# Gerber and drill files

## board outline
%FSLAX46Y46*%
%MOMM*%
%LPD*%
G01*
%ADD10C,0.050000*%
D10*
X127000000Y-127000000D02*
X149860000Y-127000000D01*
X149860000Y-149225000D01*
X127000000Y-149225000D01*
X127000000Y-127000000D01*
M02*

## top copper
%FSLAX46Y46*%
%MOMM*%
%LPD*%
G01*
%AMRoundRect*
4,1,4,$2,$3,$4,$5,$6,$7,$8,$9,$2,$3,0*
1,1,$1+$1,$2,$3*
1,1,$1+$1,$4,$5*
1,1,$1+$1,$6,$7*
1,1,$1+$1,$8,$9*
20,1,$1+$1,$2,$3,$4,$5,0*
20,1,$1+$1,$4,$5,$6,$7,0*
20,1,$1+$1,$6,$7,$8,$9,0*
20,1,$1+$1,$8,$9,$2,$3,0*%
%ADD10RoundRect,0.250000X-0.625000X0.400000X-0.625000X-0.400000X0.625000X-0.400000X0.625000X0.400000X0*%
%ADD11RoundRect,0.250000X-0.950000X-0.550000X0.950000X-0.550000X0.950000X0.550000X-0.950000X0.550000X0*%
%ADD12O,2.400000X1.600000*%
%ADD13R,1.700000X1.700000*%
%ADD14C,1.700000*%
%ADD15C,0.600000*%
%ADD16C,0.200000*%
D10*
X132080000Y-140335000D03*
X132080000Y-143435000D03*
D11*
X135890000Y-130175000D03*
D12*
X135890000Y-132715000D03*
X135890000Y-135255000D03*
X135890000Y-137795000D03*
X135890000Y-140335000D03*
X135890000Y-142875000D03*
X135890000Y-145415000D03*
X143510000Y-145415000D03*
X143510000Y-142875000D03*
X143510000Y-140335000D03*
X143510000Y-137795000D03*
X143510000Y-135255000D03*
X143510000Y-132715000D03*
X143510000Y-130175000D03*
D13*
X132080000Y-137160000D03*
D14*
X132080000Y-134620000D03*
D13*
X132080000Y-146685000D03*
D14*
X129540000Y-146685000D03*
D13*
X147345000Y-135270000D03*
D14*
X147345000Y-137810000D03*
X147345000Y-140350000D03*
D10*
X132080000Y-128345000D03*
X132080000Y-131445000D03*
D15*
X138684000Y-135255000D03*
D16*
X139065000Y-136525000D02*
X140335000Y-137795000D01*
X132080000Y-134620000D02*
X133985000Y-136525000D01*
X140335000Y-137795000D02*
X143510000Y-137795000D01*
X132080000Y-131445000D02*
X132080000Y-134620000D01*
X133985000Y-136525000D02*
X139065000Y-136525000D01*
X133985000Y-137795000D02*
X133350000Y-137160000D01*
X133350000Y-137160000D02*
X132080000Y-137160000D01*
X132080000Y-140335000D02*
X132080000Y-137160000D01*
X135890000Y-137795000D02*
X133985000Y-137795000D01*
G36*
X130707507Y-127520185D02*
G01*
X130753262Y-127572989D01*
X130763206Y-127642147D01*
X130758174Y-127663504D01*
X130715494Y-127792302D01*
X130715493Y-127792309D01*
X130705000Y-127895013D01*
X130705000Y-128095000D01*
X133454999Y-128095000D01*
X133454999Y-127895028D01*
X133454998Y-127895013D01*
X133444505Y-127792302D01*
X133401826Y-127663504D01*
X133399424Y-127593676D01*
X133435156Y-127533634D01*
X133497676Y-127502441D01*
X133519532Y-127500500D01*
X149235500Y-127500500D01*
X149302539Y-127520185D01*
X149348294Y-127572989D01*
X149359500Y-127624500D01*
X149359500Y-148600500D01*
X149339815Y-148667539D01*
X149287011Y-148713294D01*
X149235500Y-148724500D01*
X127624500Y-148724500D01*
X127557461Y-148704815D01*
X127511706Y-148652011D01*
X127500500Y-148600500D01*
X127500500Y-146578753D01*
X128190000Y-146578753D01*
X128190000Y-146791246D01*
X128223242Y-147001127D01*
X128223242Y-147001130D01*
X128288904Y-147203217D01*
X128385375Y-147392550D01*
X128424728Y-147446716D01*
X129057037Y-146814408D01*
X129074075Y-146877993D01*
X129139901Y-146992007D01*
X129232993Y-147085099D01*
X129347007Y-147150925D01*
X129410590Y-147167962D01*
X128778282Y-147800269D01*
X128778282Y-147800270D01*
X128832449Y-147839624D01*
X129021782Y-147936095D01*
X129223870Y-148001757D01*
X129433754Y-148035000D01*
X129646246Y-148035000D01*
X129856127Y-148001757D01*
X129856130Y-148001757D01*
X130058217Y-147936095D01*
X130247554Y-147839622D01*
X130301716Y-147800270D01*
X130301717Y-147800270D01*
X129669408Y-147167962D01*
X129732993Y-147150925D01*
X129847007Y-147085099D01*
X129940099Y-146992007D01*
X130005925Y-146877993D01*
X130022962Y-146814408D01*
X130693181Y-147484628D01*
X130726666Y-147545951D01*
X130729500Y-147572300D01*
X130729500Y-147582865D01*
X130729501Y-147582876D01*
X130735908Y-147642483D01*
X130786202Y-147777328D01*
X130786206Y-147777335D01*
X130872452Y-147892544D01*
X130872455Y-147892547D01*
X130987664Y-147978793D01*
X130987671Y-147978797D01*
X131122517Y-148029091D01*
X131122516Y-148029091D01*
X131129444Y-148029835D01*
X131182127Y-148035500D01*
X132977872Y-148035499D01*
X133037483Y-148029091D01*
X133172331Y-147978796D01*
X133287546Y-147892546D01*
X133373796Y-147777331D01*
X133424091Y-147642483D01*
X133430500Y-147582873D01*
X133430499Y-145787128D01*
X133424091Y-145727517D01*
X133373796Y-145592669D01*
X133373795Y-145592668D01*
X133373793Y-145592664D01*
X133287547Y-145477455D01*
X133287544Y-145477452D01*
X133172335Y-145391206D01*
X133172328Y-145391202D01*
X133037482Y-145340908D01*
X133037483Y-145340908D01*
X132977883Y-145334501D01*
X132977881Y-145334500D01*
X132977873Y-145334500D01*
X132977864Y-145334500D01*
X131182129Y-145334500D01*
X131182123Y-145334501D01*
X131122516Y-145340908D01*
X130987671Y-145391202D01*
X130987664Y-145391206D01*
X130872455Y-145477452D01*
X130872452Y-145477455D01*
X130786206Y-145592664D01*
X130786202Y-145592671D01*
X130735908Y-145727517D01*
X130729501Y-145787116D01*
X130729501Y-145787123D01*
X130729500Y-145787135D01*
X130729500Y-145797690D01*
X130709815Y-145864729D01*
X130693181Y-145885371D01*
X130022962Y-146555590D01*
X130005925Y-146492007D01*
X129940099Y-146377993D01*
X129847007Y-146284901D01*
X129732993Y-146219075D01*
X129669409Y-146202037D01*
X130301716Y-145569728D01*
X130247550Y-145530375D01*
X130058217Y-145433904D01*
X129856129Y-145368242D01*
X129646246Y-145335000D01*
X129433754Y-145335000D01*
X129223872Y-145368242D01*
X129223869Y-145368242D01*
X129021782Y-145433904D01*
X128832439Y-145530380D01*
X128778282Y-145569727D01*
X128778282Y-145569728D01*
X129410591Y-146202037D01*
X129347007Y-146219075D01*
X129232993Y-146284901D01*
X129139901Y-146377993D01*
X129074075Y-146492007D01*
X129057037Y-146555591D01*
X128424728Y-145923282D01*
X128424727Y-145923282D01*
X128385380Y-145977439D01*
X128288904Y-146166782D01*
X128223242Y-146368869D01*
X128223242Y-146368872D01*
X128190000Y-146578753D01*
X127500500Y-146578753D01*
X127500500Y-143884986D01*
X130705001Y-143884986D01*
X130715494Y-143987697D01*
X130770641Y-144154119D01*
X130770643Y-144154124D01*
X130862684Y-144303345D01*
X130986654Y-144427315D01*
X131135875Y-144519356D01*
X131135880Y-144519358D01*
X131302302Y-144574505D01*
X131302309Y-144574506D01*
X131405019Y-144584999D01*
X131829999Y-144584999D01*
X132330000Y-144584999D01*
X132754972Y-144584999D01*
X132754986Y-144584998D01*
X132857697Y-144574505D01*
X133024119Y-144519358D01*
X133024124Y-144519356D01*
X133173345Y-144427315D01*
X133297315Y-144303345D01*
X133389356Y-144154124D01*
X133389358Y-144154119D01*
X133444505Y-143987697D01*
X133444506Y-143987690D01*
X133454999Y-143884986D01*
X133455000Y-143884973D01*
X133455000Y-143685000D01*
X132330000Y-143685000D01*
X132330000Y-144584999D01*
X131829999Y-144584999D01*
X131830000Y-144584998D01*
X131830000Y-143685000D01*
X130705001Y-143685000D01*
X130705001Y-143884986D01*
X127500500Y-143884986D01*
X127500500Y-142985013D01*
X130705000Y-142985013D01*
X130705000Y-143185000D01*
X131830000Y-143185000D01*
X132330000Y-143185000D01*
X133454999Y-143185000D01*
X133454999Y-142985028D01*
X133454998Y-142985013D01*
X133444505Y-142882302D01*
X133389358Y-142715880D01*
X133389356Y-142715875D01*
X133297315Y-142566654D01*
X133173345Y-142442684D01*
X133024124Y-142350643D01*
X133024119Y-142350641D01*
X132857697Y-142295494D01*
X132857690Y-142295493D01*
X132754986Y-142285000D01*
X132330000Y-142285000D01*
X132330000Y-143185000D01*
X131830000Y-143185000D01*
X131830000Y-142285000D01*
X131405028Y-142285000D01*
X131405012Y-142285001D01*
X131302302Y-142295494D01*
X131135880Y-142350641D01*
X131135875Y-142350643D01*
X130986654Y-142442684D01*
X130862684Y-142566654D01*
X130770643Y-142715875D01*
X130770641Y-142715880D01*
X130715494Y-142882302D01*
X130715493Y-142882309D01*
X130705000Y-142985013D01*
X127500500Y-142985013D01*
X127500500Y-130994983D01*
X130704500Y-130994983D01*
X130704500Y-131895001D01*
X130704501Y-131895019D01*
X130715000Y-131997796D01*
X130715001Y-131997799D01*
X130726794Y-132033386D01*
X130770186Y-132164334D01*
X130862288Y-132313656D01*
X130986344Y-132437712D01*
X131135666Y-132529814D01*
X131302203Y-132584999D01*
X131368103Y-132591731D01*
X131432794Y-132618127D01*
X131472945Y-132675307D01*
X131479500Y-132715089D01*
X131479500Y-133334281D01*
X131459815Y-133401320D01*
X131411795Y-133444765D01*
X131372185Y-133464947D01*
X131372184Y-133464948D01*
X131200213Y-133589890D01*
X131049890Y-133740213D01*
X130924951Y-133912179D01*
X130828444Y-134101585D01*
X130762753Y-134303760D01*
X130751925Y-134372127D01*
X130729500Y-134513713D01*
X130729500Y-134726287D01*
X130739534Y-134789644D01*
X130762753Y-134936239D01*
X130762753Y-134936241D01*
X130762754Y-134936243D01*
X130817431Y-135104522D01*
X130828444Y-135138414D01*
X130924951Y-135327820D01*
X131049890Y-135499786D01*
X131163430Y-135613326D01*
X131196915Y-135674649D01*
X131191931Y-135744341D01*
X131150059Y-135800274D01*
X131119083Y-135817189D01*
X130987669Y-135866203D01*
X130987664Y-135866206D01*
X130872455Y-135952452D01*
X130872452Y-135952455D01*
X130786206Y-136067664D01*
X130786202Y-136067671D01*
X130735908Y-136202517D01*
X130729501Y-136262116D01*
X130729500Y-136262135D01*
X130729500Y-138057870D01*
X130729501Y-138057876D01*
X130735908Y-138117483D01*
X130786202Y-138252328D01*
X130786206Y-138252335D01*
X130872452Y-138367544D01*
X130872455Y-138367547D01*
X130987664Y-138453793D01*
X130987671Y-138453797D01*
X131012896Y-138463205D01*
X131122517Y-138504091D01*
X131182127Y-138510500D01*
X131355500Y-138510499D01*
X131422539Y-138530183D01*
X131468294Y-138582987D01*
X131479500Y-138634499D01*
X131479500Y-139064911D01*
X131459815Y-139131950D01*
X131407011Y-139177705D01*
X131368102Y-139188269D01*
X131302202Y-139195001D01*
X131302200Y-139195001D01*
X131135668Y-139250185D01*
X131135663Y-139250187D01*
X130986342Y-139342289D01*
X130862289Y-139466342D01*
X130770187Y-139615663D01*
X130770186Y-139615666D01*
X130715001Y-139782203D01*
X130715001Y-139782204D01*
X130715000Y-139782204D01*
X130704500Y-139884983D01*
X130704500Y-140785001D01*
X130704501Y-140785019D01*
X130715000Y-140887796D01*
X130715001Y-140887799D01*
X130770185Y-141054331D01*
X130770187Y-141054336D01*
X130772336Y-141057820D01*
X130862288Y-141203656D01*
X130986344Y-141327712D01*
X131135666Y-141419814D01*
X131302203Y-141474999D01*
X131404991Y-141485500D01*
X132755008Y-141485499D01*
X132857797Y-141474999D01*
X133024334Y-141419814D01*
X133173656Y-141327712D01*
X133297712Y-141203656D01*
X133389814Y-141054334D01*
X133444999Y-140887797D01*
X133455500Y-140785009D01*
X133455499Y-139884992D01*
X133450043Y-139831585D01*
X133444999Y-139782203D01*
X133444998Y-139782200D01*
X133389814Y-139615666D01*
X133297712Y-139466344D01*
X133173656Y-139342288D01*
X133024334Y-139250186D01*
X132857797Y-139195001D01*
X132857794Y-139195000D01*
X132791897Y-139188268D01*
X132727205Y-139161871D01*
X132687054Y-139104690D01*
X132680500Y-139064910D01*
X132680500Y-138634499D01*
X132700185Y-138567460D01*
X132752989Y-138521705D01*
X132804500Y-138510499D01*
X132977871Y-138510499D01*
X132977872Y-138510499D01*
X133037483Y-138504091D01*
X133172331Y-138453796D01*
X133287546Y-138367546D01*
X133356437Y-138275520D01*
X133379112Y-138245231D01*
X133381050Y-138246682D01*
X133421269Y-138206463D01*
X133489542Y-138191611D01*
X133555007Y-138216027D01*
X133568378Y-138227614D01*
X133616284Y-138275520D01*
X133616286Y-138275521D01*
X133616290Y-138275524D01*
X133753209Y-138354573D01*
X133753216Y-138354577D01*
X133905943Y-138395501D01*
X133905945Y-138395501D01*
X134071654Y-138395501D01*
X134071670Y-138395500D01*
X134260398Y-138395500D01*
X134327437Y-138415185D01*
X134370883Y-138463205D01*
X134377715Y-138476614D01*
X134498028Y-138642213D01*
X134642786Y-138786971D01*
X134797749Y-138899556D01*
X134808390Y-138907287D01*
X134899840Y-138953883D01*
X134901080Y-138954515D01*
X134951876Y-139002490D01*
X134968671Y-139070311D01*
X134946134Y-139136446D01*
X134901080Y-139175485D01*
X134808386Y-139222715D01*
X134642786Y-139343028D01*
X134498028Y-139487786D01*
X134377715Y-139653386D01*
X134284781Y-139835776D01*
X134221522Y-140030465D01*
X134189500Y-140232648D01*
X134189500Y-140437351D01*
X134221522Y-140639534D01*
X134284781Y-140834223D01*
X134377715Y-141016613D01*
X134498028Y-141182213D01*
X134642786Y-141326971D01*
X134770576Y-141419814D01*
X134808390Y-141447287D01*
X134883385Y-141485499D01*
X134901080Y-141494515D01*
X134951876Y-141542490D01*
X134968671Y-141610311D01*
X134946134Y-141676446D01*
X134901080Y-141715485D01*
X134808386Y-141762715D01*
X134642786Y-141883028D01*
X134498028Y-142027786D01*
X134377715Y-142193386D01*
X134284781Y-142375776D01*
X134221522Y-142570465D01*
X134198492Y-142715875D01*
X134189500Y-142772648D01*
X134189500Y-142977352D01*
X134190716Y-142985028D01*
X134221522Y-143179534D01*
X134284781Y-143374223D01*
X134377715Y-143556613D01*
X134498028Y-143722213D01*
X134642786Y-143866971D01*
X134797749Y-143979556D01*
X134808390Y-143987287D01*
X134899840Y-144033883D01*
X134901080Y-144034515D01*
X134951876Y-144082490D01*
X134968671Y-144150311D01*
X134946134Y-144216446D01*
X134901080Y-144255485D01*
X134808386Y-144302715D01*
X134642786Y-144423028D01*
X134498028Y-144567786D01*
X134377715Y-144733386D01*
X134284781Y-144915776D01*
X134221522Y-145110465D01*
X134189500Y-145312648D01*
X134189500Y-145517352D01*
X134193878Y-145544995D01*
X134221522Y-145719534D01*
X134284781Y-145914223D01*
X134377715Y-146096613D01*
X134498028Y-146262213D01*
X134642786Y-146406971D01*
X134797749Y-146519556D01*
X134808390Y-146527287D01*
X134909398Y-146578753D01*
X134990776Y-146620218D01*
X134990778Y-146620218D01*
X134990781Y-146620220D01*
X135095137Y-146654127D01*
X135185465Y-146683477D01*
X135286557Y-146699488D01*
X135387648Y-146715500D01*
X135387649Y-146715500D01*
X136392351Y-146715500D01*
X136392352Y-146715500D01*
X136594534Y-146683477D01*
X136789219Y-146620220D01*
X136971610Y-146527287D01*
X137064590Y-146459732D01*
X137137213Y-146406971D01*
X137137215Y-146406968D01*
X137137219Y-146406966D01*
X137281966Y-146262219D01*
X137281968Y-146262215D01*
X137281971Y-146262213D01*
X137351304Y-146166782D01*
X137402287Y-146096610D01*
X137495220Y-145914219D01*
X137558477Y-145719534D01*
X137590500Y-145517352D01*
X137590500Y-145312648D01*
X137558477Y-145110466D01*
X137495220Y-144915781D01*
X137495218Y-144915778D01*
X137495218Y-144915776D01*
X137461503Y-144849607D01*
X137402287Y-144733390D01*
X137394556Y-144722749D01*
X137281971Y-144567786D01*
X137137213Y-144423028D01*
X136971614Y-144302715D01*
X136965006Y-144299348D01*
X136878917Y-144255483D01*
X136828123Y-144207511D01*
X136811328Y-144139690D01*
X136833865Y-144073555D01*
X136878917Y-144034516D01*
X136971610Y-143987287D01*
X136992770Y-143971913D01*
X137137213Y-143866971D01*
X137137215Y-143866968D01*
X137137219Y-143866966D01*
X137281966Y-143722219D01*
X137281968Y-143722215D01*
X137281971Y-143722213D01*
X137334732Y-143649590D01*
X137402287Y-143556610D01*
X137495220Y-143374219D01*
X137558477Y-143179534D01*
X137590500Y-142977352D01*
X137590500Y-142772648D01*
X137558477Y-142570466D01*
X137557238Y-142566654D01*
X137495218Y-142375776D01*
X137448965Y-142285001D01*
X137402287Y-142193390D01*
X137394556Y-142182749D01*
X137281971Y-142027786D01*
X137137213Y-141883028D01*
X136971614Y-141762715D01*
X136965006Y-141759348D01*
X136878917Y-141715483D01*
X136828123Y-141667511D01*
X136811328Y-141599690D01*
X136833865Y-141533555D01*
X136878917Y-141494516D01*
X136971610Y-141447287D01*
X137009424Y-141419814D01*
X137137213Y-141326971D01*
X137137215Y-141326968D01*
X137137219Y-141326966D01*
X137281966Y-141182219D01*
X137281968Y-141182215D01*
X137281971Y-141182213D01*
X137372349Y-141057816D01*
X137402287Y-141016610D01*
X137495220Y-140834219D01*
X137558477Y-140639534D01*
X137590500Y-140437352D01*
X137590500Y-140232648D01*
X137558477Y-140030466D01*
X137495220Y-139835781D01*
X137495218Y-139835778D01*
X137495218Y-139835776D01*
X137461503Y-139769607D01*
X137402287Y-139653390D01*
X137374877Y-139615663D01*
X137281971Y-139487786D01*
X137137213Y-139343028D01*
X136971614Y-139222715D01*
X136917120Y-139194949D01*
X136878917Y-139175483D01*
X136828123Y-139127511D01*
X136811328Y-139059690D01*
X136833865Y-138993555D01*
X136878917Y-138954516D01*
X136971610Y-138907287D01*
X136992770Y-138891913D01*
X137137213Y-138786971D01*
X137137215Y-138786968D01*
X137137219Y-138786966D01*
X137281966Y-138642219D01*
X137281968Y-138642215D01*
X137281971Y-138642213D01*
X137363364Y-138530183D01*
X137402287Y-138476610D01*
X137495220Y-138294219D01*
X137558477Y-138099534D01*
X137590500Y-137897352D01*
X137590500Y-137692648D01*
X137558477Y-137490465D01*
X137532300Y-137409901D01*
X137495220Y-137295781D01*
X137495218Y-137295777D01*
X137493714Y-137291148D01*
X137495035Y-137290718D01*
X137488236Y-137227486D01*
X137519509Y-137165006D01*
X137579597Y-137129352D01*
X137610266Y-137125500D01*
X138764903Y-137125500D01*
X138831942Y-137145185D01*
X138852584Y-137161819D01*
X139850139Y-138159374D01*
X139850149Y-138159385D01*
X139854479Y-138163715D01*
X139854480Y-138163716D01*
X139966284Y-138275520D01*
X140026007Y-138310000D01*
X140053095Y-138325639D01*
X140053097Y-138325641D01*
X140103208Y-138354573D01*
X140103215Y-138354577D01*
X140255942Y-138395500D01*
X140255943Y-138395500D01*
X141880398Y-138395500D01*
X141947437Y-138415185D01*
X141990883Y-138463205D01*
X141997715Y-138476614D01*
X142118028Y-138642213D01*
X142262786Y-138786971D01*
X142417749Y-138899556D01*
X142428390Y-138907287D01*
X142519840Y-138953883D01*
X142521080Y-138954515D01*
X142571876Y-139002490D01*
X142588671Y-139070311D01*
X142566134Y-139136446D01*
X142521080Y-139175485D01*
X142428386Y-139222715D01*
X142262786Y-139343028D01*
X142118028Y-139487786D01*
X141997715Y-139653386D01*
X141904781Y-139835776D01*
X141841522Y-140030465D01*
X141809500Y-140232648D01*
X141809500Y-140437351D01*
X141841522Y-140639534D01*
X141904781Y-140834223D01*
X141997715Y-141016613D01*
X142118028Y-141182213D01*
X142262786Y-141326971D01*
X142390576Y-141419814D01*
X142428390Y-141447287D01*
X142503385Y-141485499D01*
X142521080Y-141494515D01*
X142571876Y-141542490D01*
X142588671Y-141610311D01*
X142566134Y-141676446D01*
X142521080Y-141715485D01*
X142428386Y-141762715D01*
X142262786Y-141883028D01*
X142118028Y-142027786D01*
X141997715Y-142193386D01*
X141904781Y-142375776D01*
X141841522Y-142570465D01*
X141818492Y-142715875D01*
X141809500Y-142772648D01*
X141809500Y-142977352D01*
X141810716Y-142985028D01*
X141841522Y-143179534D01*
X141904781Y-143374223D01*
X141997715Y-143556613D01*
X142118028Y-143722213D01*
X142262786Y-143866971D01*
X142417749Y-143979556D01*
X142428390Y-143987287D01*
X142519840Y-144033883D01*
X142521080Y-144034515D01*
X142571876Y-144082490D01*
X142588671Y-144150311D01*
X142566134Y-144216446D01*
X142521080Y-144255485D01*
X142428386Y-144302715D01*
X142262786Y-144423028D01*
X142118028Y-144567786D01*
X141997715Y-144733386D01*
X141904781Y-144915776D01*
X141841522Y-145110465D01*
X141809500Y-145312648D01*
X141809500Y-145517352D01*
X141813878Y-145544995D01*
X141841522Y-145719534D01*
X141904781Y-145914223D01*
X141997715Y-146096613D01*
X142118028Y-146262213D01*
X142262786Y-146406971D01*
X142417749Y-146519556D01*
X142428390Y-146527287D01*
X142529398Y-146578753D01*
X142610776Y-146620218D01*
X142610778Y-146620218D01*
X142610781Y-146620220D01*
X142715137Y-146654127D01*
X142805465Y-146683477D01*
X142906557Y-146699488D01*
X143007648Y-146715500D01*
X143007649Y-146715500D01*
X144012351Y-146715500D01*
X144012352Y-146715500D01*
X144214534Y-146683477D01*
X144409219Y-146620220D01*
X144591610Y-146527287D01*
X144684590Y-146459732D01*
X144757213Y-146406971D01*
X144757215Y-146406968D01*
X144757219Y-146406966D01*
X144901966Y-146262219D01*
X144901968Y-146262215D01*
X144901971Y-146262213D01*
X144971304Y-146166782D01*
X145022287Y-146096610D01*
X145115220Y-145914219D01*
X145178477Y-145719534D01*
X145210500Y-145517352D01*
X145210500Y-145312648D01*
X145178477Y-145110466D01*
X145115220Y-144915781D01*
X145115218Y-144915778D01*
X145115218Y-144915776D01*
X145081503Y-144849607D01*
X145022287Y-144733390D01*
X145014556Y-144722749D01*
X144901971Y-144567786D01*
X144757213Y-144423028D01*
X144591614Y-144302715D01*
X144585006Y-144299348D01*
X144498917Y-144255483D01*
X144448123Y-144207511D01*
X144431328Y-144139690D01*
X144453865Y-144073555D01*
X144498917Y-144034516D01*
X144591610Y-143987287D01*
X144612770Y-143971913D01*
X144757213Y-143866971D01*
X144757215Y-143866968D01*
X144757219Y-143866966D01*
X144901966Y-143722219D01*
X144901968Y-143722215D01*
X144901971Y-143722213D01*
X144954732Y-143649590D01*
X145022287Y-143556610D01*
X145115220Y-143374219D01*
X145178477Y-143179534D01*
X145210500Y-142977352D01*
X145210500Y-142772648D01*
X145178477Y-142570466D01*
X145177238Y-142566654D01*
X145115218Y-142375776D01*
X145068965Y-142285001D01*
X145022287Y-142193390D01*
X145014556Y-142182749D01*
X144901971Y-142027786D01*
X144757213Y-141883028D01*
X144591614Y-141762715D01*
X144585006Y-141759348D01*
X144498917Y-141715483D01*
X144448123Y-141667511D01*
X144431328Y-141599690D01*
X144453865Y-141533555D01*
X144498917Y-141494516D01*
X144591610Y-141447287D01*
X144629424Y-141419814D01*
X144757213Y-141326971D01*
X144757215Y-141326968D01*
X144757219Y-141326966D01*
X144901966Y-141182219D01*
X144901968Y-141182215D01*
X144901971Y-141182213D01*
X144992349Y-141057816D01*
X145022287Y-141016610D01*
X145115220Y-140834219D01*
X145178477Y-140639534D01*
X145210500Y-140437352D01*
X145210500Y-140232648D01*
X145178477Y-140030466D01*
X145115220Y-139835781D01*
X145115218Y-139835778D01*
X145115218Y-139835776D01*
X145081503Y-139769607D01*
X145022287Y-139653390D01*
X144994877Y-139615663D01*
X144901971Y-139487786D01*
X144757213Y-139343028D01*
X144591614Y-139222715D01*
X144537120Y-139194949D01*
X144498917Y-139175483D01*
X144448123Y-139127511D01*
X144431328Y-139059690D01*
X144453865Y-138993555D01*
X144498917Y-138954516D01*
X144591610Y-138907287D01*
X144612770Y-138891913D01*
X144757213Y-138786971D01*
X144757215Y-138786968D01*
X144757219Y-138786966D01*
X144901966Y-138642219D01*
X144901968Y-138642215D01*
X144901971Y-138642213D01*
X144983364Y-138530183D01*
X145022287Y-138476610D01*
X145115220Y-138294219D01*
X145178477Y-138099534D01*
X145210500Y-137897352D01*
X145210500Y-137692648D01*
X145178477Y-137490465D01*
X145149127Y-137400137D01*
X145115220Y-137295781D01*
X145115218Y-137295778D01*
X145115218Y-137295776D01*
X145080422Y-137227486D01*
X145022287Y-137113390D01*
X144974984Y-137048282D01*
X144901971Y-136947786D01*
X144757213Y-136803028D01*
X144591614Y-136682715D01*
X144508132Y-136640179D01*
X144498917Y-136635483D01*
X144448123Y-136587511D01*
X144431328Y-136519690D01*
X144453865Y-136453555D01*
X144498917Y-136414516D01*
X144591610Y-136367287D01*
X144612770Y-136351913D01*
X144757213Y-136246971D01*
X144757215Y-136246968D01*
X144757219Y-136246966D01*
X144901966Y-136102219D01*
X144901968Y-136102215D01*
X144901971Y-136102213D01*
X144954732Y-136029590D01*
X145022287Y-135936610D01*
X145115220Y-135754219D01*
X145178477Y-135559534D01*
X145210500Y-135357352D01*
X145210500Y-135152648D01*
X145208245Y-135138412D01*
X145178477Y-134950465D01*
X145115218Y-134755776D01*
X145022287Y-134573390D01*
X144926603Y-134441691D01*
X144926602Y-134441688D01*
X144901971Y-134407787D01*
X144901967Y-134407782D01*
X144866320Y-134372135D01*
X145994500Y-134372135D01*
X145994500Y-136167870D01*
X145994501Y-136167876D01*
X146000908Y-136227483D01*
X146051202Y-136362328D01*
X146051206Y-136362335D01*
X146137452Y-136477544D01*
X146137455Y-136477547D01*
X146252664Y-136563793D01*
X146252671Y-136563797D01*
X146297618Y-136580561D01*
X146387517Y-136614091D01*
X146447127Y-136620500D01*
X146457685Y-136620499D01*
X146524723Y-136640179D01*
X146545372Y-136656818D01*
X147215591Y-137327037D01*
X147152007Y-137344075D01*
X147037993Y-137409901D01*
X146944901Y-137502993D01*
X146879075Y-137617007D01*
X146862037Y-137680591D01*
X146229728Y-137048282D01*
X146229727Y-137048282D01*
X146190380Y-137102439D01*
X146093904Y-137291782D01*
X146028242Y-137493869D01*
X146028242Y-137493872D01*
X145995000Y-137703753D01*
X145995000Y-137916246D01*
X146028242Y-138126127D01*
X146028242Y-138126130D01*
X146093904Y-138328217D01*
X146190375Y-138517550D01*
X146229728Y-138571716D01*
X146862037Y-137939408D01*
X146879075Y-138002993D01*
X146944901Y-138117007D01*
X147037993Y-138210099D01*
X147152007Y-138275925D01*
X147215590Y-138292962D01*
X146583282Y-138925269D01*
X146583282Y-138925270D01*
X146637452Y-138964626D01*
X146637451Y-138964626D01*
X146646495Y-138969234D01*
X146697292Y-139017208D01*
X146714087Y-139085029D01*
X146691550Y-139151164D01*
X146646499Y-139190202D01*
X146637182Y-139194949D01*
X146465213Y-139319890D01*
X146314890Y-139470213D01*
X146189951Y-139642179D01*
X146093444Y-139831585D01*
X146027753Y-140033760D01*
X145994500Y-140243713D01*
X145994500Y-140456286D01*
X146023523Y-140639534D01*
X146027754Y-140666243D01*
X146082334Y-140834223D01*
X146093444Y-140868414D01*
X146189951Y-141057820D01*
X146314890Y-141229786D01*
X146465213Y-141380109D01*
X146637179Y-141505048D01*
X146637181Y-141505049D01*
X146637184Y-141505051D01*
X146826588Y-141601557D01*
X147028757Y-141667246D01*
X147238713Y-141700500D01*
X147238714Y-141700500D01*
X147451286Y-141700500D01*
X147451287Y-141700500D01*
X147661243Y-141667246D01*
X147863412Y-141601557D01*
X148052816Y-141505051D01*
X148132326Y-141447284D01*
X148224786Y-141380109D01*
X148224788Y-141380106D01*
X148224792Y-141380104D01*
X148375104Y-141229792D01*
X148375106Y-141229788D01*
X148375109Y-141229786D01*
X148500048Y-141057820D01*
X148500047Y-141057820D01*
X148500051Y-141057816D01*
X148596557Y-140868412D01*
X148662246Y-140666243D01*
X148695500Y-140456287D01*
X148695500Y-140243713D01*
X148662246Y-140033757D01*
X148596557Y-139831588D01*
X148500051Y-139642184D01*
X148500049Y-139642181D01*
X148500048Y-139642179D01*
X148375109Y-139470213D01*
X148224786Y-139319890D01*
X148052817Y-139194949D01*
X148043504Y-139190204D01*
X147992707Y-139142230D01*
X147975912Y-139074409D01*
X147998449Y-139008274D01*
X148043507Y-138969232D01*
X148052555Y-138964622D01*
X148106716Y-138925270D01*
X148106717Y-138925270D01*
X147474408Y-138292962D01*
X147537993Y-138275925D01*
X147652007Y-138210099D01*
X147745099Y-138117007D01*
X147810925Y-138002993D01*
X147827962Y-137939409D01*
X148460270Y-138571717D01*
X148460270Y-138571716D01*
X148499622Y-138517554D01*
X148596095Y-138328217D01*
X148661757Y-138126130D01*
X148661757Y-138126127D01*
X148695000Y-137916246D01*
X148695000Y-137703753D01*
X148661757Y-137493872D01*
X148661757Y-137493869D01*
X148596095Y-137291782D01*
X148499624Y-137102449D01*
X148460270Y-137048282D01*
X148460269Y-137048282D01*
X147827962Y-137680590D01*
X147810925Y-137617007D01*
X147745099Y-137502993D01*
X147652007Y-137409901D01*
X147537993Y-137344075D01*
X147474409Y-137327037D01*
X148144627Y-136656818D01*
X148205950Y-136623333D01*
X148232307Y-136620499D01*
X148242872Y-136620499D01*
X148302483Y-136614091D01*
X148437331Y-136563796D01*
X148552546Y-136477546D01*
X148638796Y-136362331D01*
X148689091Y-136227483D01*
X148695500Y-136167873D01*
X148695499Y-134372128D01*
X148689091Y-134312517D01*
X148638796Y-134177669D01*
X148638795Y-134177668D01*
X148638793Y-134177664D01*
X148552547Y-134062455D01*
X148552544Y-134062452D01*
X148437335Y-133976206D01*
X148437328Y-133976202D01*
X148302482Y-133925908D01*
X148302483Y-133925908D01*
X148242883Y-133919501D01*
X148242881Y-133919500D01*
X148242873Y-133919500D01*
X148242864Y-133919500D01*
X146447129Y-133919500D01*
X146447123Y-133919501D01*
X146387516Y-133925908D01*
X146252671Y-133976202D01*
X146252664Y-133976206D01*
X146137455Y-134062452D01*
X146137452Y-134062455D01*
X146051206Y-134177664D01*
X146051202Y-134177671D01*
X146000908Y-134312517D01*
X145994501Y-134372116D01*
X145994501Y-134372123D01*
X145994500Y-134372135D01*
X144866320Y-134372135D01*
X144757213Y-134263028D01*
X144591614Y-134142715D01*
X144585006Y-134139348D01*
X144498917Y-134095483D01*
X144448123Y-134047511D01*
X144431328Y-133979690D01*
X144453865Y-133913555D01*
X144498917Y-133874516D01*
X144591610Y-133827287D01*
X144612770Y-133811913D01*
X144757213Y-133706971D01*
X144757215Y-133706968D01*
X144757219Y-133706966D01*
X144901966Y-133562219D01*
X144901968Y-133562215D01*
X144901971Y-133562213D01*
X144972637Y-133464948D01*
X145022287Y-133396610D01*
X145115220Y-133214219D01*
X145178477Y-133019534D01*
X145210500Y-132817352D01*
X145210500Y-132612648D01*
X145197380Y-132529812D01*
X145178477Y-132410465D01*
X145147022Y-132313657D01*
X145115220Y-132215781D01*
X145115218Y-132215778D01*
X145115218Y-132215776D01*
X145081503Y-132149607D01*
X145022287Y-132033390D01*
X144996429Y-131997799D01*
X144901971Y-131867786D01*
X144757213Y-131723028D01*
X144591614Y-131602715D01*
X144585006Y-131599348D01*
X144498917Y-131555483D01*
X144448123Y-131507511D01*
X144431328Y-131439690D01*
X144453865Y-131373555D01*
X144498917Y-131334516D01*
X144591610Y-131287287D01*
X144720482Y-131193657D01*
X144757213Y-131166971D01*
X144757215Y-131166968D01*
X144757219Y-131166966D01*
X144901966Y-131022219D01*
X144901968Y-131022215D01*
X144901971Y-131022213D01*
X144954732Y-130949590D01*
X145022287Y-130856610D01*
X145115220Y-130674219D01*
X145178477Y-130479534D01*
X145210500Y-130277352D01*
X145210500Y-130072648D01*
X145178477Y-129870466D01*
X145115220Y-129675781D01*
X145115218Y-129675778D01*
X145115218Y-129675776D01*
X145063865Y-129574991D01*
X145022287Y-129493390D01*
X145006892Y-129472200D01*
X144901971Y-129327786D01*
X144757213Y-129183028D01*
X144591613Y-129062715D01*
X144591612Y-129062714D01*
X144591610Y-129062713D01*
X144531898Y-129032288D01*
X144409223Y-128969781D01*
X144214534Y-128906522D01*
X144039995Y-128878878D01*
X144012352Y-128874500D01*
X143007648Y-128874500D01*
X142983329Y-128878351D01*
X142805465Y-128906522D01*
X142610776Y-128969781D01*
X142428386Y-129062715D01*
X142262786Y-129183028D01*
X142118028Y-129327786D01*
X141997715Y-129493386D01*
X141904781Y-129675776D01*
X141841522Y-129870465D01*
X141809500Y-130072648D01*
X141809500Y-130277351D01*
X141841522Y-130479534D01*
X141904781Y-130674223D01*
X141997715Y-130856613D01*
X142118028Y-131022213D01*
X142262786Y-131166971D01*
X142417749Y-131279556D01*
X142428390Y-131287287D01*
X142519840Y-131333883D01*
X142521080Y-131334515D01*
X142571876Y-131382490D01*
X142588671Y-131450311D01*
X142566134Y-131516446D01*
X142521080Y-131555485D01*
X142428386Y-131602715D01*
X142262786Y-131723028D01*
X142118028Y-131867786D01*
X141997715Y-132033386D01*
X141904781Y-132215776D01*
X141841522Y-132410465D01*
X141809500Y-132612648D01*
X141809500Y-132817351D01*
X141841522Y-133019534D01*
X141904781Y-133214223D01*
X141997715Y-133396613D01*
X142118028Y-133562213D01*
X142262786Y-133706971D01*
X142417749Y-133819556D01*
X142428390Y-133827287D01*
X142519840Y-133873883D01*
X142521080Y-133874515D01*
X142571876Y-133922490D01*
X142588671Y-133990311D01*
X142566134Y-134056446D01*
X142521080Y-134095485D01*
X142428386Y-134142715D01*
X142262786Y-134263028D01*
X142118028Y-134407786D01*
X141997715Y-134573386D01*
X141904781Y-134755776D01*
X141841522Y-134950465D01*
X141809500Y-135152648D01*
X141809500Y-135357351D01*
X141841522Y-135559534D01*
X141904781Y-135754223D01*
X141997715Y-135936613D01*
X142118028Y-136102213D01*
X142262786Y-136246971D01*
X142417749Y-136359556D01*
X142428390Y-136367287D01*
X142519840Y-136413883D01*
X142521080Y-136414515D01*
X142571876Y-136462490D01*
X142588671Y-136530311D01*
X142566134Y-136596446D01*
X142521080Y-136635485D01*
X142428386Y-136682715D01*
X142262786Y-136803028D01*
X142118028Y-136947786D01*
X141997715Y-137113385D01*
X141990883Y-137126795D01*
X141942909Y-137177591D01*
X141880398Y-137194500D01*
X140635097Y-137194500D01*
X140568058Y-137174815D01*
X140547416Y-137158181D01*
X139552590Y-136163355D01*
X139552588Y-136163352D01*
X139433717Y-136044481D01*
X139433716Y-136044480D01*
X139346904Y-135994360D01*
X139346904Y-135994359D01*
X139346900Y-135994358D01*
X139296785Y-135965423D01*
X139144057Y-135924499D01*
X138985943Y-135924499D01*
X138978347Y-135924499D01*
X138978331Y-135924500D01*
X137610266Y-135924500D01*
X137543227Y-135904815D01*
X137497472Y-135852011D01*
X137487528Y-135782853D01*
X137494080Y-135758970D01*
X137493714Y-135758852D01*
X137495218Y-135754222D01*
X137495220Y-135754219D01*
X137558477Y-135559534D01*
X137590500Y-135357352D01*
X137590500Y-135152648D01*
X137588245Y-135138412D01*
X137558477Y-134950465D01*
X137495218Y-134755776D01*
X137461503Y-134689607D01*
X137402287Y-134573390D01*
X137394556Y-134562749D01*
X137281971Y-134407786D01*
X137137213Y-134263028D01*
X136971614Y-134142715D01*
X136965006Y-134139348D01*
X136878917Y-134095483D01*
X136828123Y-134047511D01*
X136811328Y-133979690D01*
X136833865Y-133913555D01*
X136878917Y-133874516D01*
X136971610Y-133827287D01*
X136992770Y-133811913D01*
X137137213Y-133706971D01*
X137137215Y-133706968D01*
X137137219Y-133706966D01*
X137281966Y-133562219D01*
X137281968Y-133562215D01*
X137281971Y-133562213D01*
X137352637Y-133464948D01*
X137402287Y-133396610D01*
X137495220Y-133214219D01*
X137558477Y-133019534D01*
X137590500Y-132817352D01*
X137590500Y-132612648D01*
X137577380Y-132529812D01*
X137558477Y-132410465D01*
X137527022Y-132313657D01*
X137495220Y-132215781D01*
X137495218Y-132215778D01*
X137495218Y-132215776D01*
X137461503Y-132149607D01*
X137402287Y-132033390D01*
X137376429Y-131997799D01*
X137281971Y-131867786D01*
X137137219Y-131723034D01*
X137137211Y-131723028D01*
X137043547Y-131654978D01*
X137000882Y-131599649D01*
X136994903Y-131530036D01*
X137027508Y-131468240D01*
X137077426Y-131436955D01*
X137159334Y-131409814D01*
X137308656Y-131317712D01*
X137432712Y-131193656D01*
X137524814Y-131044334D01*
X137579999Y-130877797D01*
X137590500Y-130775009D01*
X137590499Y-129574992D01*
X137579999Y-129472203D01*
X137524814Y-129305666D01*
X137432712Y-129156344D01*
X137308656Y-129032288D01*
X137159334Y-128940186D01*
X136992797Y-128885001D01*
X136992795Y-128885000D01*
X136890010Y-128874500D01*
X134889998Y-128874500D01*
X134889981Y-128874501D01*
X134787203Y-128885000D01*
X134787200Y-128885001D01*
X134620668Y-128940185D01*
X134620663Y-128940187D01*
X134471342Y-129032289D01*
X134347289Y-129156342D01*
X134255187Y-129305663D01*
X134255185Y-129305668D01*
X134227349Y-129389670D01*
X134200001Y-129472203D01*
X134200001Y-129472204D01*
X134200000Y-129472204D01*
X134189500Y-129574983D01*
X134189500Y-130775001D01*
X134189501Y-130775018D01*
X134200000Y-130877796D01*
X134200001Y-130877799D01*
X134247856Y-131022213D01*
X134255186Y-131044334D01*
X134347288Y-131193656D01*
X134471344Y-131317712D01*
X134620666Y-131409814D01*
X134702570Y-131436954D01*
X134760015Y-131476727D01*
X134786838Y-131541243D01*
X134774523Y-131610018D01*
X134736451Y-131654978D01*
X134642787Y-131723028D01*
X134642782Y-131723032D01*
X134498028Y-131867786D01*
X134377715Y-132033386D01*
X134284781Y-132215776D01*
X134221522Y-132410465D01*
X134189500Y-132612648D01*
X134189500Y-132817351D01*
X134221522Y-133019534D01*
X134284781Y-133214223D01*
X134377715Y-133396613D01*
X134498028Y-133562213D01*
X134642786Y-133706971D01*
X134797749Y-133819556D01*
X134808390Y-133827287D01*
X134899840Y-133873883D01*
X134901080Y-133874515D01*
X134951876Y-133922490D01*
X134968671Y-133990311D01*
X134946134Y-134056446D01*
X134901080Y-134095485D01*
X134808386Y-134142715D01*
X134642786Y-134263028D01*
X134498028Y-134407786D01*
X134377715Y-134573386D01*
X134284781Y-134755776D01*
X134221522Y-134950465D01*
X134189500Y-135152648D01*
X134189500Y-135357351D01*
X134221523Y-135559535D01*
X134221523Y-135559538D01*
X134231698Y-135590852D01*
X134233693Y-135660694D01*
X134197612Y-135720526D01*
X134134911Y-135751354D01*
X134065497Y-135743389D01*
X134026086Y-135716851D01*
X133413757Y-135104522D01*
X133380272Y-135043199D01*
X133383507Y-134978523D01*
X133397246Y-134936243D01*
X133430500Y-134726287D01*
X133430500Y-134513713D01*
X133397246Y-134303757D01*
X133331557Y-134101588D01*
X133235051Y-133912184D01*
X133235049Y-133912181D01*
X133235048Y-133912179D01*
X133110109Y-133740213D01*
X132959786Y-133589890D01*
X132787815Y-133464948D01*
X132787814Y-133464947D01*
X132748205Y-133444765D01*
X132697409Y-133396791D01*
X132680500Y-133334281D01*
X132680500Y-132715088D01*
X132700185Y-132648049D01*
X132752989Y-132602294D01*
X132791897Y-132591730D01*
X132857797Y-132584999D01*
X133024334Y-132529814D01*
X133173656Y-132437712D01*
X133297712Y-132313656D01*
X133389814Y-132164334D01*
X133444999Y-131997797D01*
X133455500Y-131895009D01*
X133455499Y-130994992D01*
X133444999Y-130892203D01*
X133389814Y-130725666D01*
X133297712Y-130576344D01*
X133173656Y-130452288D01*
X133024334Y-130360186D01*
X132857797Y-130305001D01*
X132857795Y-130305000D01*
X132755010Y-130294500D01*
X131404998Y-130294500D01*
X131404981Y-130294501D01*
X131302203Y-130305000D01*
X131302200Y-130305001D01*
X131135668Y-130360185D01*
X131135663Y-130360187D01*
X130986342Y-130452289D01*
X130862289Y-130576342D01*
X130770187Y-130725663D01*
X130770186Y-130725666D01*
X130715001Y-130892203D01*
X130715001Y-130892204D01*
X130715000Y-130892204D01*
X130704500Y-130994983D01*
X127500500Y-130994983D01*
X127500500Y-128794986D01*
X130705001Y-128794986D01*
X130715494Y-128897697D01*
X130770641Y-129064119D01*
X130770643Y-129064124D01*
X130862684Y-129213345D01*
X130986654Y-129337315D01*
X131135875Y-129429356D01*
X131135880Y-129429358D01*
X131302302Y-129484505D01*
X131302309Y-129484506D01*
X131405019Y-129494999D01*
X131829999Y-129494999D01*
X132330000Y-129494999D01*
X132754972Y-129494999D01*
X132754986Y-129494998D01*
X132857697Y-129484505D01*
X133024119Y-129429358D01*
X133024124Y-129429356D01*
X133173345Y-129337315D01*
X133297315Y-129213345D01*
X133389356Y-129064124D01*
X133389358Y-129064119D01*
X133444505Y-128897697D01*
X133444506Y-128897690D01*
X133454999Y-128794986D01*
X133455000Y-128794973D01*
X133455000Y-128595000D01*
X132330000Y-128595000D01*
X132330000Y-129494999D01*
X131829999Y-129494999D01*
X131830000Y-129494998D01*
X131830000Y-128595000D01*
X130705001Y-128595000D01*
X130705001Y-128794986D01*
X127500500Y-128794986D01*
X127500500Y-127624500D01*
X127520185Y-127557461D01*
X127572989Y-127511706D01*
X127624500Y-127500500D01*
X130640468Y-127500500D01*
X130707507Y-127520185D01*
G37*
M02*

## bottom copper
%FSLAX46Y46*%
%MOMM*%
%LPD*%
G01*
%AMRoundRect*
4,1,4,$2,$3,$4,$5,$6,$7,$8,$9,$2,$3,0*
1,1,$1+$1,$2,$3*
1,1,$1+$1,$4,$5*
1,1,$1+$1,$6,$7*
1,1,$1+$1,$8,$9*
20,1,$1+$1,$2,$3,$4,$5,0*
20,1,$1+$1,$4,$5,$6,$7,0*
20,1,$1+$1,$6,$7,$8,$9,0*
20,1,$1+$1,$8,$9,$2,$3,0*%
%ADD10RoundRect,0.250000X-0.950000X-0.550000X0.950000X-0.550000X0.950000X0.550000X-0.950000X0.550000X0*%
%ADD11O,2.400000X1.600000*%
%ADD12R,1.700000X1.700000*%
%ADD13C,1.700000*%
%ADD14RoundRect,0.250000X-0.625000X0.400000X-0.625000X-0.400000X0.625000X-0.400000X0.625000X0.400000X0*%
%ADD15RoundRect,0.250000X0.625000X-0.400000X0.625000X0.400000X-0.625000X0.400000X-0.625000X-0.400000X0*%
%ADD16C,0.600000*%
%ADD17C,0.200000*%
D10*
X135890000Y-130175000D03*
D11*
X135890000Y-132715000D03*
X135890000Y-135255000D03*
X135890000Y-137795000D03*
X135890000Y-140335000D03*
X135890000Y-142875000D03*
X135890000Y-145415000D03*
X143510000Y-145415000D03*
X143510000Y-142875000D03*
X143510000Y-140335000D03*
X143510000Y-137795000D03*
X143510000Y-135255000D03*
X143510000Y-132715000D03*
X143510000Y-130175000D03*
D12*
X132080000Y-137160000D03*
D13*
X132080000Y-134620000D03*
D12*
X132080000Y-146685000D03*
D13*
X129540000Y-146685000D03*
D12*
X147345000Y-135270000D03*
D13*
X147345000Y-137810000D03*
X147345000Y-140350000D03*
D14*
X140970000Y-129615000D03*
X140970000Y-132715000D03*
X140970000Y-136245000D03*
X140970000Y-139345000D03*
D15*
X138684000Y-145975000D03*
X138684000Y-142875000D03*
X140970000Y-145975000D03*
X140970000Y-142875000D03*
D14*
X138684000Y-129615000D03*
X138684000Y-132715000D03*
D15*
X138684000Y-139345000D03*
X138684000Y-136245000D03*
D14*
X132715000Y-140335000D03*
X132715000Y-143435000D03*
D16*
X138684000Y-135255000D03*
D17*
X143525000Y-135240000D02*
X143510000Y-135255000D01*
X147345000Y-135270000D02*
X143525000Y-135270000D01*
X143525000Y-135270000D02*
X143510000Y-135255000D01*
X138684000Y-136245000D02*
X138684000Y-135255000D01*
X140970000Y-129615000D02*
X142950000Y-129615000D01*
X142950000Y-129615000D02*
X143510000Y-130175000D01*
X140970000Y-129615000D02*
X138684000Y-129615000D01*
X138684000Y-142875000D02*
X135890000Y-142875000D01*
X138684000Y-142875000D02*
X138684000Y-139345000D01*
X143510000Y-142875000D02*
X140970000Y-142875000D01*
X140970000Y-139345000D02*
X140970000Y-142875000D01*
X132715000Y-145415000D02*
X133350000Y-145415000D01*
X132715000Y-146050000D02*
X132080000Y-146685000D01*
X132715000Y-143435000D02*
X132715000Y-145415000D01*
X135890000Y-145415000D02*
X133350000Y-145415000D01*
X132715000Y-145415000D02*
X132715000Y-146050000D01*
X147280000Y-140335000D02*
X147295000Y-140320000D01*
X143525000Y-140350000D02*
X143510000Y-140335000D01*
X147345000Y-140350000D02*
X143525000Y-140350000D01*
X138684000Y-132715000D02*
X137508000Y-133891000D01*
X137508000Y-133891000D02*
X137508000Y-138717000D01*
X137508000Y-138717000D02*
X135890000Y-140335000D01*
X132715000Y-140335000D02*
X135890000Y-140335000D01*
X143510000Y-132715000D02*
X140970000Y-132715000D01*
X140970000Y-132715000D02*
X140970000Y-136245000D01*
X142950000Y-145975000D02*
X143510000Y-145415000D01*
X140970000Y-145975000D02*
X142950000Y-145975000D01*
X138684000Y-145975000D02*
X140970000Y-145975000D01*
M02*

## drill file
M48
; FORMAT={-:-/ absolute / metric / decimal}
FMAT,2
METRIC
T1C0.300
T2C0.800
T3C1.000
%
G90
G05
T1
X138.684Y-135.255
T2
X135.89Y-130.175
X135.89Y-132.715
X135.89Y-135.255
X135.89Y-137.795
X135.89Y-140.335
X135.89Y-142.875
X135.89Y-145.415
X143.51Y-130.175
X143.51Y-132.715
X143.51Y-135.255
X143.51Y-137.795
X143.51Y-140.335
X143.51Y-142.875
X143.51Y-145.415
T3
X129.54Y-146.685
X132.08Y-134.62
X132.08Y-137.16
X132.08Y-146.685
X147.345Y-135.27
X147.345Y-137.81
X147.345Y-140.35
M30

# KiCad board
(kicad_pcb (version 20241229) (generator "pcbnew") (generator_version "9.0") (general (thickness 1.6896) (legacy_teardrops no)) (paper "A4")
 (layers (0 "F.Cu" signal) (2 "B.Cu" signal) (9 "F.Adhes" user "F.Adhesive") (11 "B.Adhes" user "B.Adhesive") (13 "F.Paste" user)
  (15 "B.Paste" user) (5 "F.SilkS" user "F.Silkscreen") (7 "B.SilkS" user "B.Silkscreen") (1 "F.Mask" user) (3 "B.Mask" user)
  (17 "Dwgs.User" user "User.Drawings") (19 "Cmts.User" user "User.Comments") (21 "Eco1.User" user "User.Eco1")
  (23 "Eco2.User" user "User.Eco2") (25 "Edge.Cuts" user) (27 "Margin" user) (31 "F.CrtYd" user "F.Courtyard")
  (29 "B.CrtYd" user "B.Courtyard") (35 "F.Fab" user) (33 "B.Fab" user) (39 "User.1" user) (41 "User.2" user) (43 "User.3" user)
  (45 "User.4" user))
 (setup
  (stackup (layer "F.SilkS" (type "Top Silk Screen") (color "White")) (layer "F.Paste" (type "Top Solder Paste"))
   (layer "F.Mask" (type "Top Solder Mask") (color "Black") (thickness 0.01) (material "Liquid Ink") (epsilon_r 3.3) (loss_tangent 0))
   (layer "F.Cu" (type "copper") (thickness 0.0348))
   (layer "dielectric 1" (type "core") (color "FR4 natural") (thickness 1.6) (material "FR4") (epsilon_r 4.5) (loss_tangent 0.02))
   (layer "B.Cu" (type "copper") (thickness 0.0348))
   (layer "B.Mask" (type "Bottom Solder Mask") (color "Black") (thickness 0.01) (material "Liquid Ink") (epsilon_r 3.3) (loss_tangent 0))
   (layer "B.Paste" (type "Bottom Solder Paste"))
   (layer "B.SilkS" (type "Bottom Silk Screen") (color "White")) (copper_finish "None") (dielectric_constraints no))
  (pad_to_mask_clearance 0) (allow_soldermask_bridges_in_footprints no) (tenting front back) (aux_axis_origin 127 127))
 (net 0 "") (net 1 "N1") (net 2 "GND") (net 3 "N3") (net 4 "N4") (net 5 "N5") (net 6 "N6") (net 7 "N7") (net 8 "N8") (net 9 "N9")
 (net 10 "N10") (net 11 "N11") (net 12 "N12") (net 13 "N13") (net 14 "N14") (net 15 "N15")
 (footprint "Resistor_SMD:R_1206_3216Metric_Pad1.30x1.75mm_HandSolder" (layer "F.Cu") (at 132.08 141.885 -90)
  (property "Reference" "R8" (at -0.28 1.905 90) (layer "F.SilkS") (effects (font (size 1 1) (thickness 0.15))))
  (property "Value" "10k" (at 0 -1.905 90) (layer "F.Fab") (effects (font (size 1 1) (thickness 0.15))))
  (pad "1" smd roundrect (at -1.55 0 270) (size 1.3 1.75) (layers "F.Cu" "F.Mask" "F.Paste") (roundrect_rratio 0.192308) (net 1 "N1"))
  (pad "2" smd roundrect (at 1.55 0 270) (size 1.3 1.75) (layers "F.Cu" "F.Mask" "F.Paste") (roundrect_rratio 0.192308) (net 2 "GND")))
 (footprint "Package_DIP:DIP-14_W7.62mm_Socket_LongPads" (layer "F.Cu") (at 135.89 130.175)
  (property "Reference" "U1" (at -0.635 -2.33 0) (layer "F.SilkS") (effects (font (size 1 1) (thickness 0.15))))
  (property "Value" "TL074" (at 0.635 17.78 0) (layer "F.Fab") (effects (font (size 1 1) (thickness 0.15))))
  (pad "1" thru_hole roundrect (at 0 0) (size 2.4 1.6) (drill 0.8) (layers "*.Cu" "*.Mask") (remove_unused_layers no)
   (roundrect_rratio 0.15625) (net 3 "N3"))
  (pad "2" thru_hole oval (at 0 2.54) (size 2.4 1.6) (drill 0.8) (layers "*.Cu" "*.Mask") (remove_unused_layers no) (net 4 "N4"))
  (pad "3" thru_hole oval (at 0 5.08) (size 2.4 1.6) (drill 0.8) (layers "*.Cu" "*.Mask") (remove_unused_layers no) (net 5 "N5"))
  (pad "4" thru_hole oval (at 0 7.62) (size 2.4 1.6) (drill 0.8) (layers "*.Cu" "*.Mask") (remove_unused_layers no) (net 1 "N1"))
  (pad "5" thru_hole oval (at 0 10.16) (size 2.4 1.6) (drill 0.8) (layers "*.Cu" "*.Mask") (remove_unused_layers no) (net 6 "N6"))
  (pad "6" thru_hole oval (at 0 12.7) (size 2.4 1.6) (drill 0.8) (layers "*.Cu" "*.Mask") (remove_unused_layers no) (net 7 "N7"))
  (pad "7" thru_hole oval (at 0 15.24) (size 2.4 1.6) (drill 0.8) (layers "*.Cu" "*.Mask") (remove_unused_layers no) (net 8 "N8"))
  (pad "8" thru_hole oval (at 7.62 15.24) (size 2.4 1.6) (drill 0.8) (layers "*.Cu" "*.Mask") (remove_unused_layers no) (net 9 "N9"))
  (pad "9" thru_hole oval (at 7.62 12.7) (size 2.4 1.6) (drill 0.8) (layers "*.Cu" "*.Mask") (remove_unused_layers no) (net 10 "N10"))
  (pad "10" thru_hole oval (at 7.62 10.16) (size 2.4 1.6) (drill 0.8) (layers "*.Cu" "*.Mask") (remove_unused_layers no) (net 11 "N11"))
  (pad "11" thru_hole oval (at 7.62 7.62) (size 2.4 1.6) (drill 0.8) (layers "*.Cu" "*.Mask") (remove_unused_layers no) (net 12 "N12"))
  (pad "12" thru_hole oval (at 7.62 5.08) (size 2.4 1.6) (drill 0.8) (layers "*.Cu" "*.Mask") (remove_unused_layers no) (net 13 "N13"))
  (pad "13" thru_hole oval (at 7.62 2.54) (size 2.4 1.6) (drill 0.8) (layers "*.Cu" "*.Mask") (remove_unused_layers no) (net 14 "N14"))
  (pad "14" thru_hole oval (at 7.62 0) (size 2.4 1.6) (drill 0.8) (layers "*.Cu" "*.Mask") (remove_unused_layers no) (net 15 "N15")))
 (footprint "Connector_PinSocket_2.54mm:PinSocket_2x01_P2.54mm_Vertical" (layer "F.Cu") (at 132.08 137.16 -90)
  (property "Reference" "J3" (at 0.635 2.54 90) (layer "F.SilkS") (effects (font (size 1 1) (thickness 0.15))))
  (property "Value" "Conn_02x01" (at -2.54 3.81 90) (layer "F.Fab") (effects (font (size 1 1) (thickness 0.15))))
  (pad "1" thru_hole rect (at 0 0 270) (size 1.7 1.7) (drill 1) (layers "*.Cu" "*.Mask") (remove_unused_layers no) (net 1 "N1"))
  (pad "2" thru_hole circle (at -2.54 0 270) (size 1.7 1.7) (drill 1) (layers "*.Cu" "*.Mask") (remove_unused_layers no) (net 12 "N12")))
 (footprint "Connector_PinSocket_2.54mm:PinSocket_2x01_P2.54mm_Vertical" (layer "F.Cu") (at 132.08 146.685)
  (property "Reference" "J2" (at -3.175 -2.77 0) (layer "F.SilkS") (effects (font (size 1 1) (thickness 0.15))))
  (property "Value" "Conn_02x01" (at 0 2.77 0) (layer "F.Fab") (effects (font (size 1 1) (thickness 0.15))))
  (pad "1" thru_hole rect (at 0 0) (size 1.7 1.7) (drill 1) (layers "*.Cu" "*.Mask") (remove_unused_layers no) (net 8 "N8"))
  (pad "2" thru_hole circle (at -2.54 0) (size 1.7 1.7) (drill 1) (layers "*.Cu" "*.Mask") (remove_unused_layers no) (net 2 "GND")))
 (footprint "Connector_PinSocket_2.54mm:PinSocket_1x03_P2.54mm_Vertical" (layer "F.Cu") (at 147.345 135.27)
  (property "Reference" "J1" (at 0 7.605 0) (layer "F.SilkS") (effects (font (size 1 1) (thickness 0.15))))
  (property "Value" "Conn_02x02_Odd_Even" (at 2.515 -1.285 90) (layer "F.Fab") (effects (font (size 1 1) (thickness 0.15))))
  (pad "1" thru_hole rect (at 0 0) (size 1.7 1.7) (drill 1) (layers "*.Cu" "*.Mask") (remove_unused_layers no) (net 13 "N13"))
  (pad "2" thru_hole circle (at 0 2.54) (size 1.7 1.7) (drill 1) (layers "*.Cu" "*.Mask") (remove_unused_layers no) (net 2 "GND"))
  (pad "3" thru_hole circle (at 0 5.08) (size 1.7 1.7) (drill 1) (layers "*.Cu" "*.Mask") (remove_unused_layers no) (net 11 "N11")))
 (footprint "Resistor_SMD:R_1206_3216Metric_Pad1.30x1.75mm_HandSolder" (layer "F.Cu") (at 132.08 129.895 -90)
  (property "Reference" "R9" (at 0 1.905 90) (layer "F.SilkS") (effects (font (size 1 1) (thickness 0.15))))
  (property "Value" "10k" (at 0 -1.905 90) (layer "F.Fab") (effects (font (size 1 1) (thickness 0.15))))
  (pad "1" smd roundrect (at -1.55 0 270) (size 1.3 1.75) (layers "F.Cu" "F.Mask" "F.Paste") (roundrect_rratio 0.192308) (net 2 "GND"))
  (pad "2" smd roundrect (at 1.55 0 270) (size 1.3 1.75) (layers "F.Cu" "F.Mask" "F.Paste") (roundrect_rratio 0.192308) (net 12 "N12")))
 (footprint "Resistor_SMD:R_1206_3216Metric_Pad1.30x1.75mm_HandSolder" (layer "B.Cu") (at 140.97 131.165 -90)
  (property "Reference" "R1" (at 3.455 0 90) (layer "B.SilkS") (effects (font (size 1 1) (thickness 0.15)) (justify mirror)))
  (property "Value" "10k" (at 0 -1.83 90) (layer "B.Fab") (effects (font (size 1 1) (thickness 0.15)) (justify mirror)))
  (pad "1" smd roundrect (at -1.55 0 270) (size 1.3 1.75) (layers "B.Cu" "B.Mask" "B.Paste") (roundrect_rratio 0.192308) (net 15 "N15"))
  (pad "2" smd roundrect (at 1.55 0 270) (size 1.3 1.75) (layers "B.Cu" "B.Mask" "B.Paste") (roundrect_rratio 0.192308) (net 14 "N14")))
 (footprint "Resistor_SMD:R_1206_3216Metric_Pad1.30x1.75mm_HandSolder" (layer "B.Cu") (at 140.97 137.795 -90)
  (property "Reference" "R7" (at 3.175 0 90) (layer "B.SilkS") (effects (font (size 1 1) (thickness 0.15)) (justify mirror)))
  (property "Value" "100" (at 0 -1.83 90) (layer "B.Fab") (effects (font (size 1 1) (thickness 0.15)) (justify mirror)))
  (pad "1" smd roundrect (at -1.55 0 270) (size 1.3 1.75) (layers "B.Cu" "B.Mask" "B.Paste") (roundrect_rratio 0.192308) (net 14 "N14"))
  (pad "2" smd roundrect (at 1.55 0 270) (size 1.3 1.75) (layers "B.Cu" "B.Mask" "B.Paste") (roundrect_rratio 0.192308) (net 10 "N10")))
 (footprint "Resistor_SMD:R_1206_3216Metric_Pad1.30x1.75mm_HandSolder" (layer "B.Cu") (at 138.684 144.425 90)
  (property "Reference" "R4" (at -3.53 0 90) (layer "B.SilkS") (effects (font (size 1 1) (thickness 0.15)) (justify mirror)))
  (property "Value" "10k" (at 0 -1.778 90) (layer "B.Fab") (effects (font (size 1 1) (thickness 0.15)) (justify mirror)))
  (pad "1" smd roundrect (at -1.55 0 90) (size 1.3 1.75) (layers "B.Cu" "B.Mask" "B.Paste") (roundrect_rratio 0.192308) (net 9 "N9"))
  (pad "2" smd roundrect (at 1.55 0 90) (size 1.3 1.75) (layers "B.Cu" "B.Mask" "B.Paste") (roundrect_rratio 0.192308) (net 7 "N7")))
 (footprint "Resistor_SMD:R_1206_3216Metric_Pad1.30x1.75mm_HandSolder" (layer "B.Cu") (at 140.97 144.425 90)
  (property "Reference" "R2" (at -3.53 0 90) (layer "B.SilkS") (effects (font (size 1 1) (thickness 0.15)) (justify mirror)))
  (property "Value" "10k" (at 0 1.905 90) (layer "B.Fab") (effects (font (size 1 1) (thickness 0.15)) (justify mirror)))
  (pad "1" smd roundrect (at -1.55 0 90) (size 1.3 1.75) (layers "B.Cu" "B.Mask" "B.Paste") (roundrect_rratio 0.192308) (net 9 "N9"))
  (pad "2" smd roundrect (at 1.55 0 90) (size 1.3 1.75) (layers "B.Cu" "B.Mask" "B.Paste") (roundrect_rratio 0.192308) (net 10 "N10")))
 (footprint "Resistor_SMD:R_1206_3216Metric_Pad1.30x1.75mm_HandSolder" (layer "B.Cu") (at 138.684 131.165 -90)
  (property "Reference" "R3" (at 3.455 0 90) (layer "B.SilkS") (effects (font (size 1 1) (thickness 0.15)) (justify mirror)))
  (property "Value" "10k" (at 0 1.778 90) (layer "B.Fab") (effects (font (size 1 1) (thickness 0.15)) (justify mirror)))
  (pad "1" smd roundrect (at -1.55 0 270) (size 1.3 1.75) (layers "B.Cu" "B.Mask" "B.Paste") (roundrect_rratio 0.192308) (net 15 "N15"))
  (pad "2" smd roundrect (at 1.55 0 270) (size 1.3 1.75) (layers "B.Cu" "B.Mask" "B.Paste") (roundrect_rratio 0.192308) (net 6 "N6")))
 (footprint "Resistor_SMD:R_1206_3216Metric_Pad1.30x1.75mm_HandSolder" (layer "B.Cu") (at 138.684 137.795 90)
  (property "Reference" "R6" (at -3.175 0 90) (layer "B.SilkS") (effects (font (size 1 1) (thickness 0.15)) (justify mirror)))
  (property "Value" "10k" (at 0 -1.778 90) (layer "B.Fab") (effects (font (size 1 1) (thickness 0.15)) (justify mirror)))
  (pad "1" smd roundrect (at -1.55 0 90) (size 1.3 1.75) (layers "B.Cu" "B.Mask" "B.Paste") (roundrect_rratio 0.192308) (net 7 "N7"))
  (pad "2" smd roundrect (at 1.55 0 90) (size 1.3 1.75) (layers "B.Cu" "B.Mask" "B.Paste") (roundrect_rratio 0.192308) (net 2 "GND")))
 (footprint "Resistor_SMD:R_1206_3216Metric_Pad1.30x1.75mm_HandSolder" (layer "B.Cu") (at 132.715 141.885 -90)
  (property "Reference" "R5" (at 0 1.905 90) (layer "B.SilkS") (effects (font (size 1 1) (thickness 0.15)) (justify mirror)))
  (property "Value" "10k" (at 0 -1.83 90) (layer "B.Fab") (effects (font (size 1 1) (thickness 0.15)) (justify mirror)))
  (pad "1" smd roundrect (at -1.55 0 270) (size 1.3 1.75) (layers "B.Cu" "B.Mask" "B.Paste") (roundrect_rratio 0.192308) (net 6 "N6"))
  (pad "2" smd roundrect (at 1.55 0 270) (size 1.3 1.75) (layers "B.Cu" "B.Mask" "B.Paste") (roundrect_rratio 0.192308) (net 8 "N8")))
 (gr_rect (start 127 127) (end 149.86 149.225) (stroke (width 0.05) (type default)) (fill no) (layer "Edge.Cuts"))
 (segment (start 143.525 135.24) (end 143.51 135.255) (width 0.2) (layer "B.Cu") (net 13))
 (segment (start 147.345 135.27) (end 143.525 135.27) (width 0.2) (layer "B.Cu") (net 13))
 (segment (start 143.525 135.27) (end 143.51 135.255) (width 0.2) (layer "B.Cu") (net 13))
 (via (at 138.684 135.255) (size 0.6) (drill 0.3) (layers "F.Cu" "B.Cu") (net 2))
 (segment (start 138.684 136.245) (end 138.684 135.255) (width 0.2) (layer "B.Cu") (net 2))
 (segment (start 140.97 129.615) (end 142.95 129.615) (width 0.2) (layer "B.Cu") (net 15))
 (segment (start 142.95 129.615) (end 143.51 130.175) (width 0.2) (layer "B.Cu") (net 15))
 (segment (start 140.97 129.615) (end 138.684 129.615) (width 0.2) (layer "B.Cu") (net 15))
 (segment (start 138.684 142.875) (end 135.89 142.875) (width 0.2) (layer "B.Cu") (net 7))
 (segment (start 138.684 142.875) (end 138.684 139.345) (width 0.2) (layer "B.Cu") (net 7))
 (segment (start 143.51 142.875) (end 140.97 142.875) (width 0.2) (layer "B.Cu") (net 10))
 (segment (start 140.97 139.345) (end 140.97 142.875) (width 0.2) (layer "B.Cu") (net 10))
 (segment (start 132.715 145.415) (end 133.35 145.415) (width 0.2) (layer "B.Cu") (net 8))
 (segment (start 132.715 146.05) (end 132.08 146.685) (width 0.2) (layer "B.Cu") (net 8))
 (segment (start 132.715 143.435) (end 132.715 145.415) (width 0.2) (layer "B.Cu") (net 8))
 (segment (start 135.89 145.415) (end 133.35 145.415) (width 0.2) (layer "B.Cu") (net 8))
 (segment (start 132.715 145.415) (end 132.715 146.05) (width 0.2) (layer "B.Cu") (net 8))
 (segment (start 139.065 136.525) (end 140.335 137.795) (width 0.2) (layer "F.Cu") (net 12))
 (segment (start 132.08 134.62) (end 133.985 136.525) (width 0.2) (layer "F.Cu") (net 12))
 (segment (start 140.335 137.795) (end 143.51 137.795) (width 0.2) (layer "F.Cu") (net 12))
 (segment (start 132.08 131.445) (end 132.08 134.62) (width 0.2) (layer "F.Cu") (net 12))
 (segment (start 133.985 136.525) (end 139.065 136.525) (width 0.2) (layer "F.Cu") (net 12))
 (segment (start 133.985 137.795) (end 133.35 137.16) (width 0.2) (layer "F.Cu") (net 1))
 (segment (start 133.35 137.16) (end 132.08 137.16) (width 0.2) (layer "F.Cu") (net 1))
 (segment (start 132.08 140.335) (end 132.08 137.16) (width 0.2) (layer "F.Cu") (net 1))
 (segment (start 135.89 137.795) (end 133.985 137.795) (width 0.2) (layer "F.Cu") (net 1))
 (segment (start 147.28 140.335) (end 147.295 140.32) (width 0.2) (layer "B.Cu") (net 11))
 (segment (start 143.525 140.35) (end 143.51 140.335) (width 0.2) (layer "B.Cu") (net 11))
 (segment (start 147.345 140.35) (end 143.525 140.35) (width 0.2) (layer "B.Cu") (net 11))
 (segment (start 138.684 132.715) (end 137.508 133.891) (width 0.2) (layer "B.Cu") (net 6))
 (segment (start 137.508 133.891) (end 137.508 138.717) (width 0.2) (layer "B.Cu") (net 6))
 (segment (start 137.508 138.717) (end 135.89 140.335) (width 0.2) (layer "B.Cu") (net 6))
 (segment (start 132.715 140.335) (end 135.89 140.335) (width 0.2) (layer "B.Cu") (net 6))
 (segment (start 143.51 132.715) (end 140.97 132.715) (width 0.2) (layer "B.Cu") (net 14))
 (segment (start 140.97 132.715) (end 140.97 136.245) (width 0.2) (layer "B.Cu") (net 14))
 (segment (start 142.95 145.975) (end 143.51 145.415) (width 0.2) (layer "B.Cu") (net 9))
 (segment (start 140.97 145.975) (end 142.95 145.975) (width 0.2) (layer "B.Cu") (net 9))
 (segment (start 138.684 145.975) (end 140.97 145.975) (width 0.2) (layer "B.Cu") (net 9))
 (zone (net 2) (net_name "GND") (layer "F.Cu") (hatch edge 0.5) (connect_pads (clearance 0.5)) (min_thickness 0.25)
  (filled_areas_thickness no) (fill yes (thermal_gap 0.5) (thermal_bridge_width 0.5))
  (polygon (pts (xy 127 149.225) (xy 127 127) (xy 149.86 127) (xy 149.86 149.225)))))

